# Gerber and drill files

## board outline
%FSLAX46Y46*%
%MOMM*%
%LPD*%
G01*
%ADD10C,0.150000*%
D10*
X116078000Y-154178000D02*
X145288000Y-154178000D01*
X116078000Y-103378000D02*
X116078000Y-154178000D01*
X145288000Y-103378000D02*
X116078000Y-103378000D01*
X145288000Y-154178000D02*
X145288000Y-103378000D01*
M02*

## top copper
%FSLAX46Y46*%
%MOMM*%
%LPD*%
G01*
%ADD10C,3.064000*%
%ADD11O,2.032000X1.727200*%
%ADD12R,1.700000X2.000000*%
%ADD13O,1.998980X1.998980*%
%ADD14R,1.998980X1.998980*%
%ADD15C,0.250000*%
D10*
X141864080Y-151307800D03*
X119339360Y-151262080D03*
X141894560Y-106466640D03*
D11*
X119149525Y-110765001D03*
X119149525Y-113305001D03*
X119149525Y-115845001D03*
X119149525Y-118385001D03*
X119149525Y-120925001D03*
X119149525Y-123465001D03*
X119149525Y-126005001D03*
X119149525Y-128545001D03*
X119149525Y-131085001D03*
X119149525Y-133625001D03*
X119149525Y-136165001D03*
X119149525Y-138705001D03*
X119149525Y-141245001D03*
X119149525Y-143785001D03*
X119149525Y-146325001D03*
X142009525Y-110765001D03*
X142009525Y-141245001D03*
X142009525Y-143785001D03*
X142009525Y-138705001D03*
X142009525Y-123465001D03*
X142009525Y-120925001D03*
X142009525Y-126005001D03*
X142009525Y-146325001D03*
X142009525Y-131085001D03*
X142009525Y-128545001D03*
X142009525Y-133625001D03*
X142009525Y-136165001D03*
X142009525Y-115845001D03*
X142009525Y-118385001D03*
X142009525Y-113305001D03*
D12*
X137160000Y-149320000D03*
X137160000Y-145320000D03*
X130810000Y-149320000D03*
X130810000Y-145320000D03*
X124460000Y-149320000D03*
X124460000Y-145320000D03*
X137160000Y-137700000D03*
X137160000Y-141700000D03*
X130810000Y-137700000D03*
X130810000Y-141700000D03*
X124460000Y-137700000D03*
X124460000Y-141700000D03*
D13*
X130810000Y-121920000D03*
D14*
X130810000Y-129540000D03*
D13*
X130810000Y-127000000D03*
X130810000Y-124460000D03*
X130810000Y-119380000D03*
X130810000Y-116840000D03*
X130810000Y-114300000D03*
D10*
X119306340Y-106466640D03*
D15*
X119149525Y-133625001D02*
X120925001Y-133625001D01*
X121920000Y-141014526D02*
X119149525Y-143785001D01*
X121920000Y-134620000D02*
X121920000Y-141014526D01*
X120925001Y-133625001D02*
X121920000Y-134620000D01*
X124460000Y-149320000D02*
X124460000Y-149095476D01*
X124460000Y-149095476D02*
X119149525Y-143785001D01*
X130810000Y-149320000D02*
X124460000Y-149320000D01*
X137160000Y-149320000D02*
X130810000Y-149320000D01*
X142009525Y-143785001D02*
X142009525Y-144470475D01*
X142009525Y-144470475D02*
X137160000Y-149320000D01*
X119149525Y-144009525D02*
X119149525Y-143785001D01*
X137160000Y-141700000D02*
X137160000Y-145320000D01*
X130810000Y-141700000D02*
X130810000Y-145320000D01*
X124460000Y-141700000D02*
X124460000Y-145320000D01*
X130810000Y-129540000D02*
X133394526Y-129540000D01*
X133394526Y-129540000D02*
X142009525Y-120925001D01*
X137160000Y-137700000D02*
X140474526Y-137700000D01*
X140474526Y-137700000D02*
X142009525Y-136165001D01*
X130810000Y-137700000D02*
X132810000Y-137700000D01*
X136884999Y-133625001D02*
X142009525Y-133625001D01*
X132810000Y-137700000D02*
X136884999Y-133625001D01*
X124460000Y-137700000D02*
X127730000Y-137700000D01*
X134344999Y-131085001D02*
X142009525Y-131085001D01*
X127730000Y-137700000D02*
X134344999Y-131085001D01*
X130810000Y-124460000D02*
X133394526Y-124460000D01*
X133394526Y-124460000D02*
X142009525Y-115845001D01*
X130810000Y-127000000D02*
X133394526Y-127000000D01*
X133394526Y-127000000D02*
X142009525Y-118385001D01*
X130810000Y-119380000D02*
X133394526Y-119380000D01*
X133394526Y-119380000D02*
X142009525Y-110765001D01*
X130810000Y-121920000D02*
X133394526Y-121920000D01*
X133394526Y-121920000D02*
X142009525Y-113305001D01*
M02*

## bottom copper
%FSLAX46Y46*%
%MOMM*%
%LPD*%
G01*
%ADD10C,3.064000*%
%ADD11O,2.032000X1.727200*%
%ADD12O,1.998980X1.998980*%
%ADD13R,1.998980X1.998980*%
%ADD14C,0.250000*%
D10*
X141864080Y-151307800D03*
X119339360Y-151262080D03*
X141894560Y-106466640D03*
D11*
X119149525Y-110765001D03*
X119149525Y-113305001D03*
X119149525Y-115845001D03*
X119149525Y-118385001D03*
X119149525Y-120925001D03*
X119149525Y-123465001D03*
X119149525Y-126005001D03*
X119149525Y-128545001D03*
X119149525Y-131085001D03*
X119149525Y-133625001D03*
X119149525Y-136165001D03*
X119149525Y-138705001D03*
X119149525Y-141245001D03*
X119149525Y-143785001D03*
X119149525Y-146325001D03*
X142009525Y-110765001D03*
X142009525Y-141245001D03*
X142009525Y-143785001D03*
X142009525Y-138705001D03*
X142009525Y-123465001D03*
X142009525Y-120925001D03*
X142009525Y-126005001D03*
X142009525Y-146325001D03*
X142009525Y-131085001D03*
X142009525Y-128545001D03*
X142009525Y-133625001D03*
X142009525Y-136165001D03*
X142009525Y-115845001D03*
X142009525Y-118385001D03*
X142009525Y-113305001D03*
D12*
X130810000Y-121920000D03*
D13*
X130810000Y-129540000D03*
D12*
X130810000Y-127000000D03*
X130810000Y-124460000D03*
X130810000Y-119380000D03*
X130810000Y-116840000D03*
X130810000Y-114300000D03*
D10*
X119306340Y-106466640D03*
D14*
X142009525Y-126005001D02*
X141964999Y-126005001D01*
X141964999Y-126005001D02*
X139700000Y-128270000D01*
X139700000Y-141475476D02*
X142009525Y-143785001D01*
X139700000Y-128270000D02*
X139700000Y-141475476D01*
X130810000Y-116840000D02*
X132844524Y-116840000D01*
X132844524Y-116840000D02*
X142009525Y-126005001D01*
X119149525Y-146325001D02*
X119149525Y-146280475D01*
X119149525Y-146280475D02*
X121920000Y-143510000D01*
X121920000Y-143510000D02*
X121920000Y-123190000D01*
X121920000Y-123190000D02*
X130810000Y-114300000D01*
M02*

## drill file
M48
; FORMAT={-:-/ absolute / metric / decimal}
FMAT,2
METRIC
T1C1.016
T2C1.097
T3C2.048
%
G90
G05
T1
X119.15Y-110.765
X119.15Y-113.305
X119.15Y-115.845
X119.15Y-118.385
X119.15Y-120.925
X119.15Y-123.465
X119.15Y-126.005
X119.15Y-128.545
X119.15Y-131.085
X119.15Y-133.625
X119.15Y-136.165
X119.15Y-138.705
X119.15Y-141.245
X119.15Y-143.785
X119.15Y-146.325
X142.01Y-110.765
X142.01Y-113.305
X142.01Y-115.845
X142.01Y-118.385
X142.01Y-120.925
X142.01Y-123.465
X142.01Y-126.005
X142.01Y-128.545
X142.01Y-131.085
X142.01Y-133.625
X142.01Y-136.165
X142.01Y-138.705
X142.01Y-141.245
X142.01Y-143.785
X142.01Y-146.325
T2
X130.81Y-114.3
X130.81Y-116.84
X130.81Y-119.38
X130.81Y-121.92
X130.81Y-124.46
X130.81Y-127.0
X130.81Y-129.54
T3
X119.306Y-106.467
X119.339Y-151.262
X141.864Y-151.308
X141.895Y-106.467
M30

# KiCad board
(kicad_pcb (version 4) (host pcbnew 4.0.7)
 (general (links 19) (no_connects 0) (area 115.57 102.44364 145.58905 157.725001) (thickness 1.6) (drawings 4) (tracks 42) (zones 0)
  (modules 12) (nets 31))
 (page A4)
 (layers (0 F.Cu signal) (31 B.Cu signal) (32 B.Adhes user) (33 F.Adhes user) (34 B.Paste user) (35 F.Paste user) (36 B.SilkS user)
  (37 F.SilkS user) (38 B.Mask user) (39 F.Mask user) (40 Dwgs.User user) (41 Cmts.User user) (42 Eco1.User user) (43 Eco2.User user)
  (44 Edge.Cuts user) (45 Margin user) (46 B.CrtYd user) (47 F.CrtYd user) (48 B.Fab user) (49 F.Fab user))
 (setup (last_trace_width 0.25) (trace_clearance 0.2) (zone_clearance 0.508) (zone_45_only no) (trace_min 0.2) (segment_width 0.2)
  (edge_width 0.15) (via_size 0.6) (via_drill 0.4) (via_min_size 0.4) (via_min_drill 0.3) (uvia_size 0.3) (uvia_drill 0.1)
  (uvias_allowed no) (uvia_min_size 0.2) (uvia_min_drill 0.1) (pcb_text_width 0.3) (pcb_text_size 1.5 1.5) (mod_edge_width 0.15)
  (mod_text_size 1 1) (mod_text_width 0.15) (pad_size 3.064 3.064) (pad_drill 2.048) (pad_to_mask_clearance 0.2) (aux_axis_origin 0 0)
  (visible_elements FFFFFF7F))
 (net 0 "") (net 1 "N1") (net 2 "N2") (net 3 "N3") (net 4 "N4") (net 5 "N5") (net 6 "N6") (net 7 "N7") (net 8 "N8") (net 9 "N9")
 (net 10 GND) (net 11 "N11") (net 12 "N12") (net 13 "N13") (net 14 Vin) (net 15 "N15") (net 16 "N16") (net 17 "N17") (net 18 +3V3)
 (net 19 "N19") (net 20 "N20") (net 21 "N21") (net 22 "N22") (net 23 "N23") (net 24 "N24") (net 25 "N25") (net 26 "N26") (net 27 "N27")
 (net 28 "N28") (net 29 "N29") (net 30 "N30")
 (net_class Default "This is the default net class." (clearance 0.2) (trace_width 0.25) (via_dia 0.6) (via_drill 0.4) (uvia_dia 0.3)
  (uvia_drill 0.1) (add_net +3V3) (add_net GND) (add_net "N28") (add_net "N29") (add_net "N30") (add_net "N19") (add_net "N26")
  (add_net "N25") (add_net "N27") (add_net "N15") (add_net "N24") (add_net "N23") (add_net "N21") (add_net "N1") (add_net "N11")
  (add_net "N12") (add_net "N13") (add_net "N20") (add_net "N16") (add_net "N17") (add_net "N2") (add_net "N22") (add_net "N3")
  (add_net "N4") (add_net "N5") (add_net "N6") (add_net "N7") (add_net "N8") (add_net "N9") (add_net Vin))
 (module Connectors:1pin (layer F.Cu) (at 141.86408 151.3078)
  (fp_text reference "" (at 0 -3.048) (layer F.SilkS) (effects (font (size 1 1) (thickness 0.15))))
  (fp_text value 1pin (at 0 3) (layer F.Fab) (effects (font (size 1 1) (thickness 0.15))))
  (pad 1 thru_hole circle (at 0 0) (size 3.064 3.064) (drill 2.048) (layers *.Cu *.Mask)))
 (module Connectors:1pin (layer F.Cu) (at 119.33936 151.26208)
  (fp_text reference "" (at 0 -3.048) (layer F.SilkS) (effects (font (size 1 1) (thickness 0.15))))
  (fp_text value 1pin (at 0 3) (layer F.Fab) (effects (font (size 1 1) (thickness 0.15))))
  (pad 1 thru_hole circle (at 0 0) (size 3.064 3.064) (drill 2.048) (layers *.Cu *.Mask)))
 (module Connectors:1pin (layer F.Cu) (at 141.89456 106.46664)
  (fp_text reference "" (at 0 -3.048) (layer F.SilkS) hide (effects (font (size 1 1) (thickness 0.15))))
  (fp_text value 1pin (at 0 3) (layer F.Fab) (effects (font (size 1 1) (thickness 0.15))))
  (pad 1 thru_hole circle (at 0 0) (size 3.064 3.064) (drill 2.048) (layers *.Cu *.Mask)))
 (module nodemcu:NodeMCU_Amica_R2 (layer F.Cu) (at 119.149525 110.765001)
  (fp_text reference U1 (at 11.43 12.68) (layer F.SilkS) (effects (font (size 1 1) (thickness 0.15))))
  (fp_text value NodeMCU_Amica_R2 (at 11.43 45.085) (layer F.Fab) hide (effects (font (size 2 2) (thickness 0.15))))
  (pad 1 thru_hole oval (at 0 0) (size 2.032 1.7272) (drill 1.016) (layers *.Cu *.Mask F.SilkS) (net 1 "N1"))
  (pad 2 thru_hole oval (at 0 2.54) (size 2.032 1.7272) (drill 1.016) (layers *.Cu *.Mask F.SilkS) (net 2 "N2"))
  (pad 3 thru_hole oval (at 0 5.08) (size 2.032 1.7272) (drill 1.016) (layers *.Cu *.Mask F.SilkS) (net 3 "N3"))
  (pad 4 thru_hole oval (at 0 7.62) (size 2.032 1.7272) (drill 1.016) (layers *.Cu *.Mask F.SilkS) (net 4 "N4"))
  (pad 5 thru_hole oval (at 0 10.16) (size 2.032 1.7272) (drill 1.016) (layers *.Cu *.Mask F.SilkS) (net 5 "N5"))
  (pad 6 thru_hole oval (at 0 12.7) (size 2.032 1.7272) (drill 1.016) (layers *.Cu *.Mask F.SilkS) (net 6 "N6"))
  (pad 7 thru_hole oval (at 0 15.24) (size 2.032 1.7272) (drill 1.016) (layers *.Cu *.Mask F.SilkS) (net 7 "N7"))
  (pad 8 thru_hole oval (at 0 17.78) (size 2.032 1.7272) (drill 1.016) (layers *.Cu *.Mask F.SilkS) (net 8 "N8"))
  (pad 9 thru_hole oval (at 0 20.32) (size 2.032 1.7272) (drill 1.016) (layers *.Cu *.Mask F.SilkS) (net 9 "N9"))
  (pad 10 thru_hole oval (at 0 22.86) (size 2.032 1.7272) (drill 1.016) (layers *.Cu *.Mask F.SilkS) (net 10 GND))
  (pad 11 thru_hole oval (at 0 25.4) (size 2.032 1.7272) (drill 1.016) (layers *.Cu *.Mask F.SilkS) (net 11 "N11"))
  (pad 12 thru_hole oval (at 0 27.94) (size 2.032 1.7272) (drill 1.016) (layers *.Cu *.Mask F.SilkS) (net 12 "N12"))
  (pad 13 thru_hole oval (at 0 30.48) (size 2.032 1.7272) (drill 1.016) (layers *.Cu *.Mask F.SilkS) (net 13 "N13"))
  (pad 14 thru_hole oval (at 0 33.02) (size 2.032 1.7272) (drill 1.016) (layers *.Cu *.Mask F.SilkS) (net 10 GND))
  (pad 15 thru_hole oval (at 0 35.56) (size 2.032 1.7272) (drill 1.016) (layers *.Cu *.Mask F.SilkS) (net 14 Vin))
  (pad 30 thru_hole oval (at 22.86 0) (size 2.032 1.7272) (drill 1.016) (layers *.Cu *.Mask F.SilkS) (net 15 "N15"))
  (pad 18 thru_hole oval (at 22.86 30.48) (size 2.032 1.7272) (drill 1.016) (layers *.Cu *.Mask F.SilkS) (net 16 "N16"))
  (pad 17 thru_hole oval (at 22.86 33.02) (size 2.032 1.7272) (drill 1.016) (layers *.Cu *.Mask F.SilkS) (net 10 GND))
  (pad 19 thru_hole oval (at 22.86 27.94) (size 2.032 1.7272) (drill 1.016) (layers *.Cu *.Mask F.SilkS) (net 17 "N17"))
  (pad 25 thru_hole oval (at 22.86 12.7) (size 2.032 1.7272) (drill 1.016) (layers *.Cu *.Mask F.SilkS) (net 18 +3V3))
  (pad 26 thru_hole oval (at 22.86 10.16) (size 2.032 1.7272) (drill 1.016) (layers *.Cu *.Mask F.SilkS) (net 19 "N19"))
  (pad 24 thru_hole oval (at 22.86 15.24) (size 2.032 1.7272) (drill 1.016) (layers *.Cu *.Mask F.SilkS) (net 10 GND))
  (pad 16 thru_hole oval (at 22.86 35.56) (size 2.032 1.7272) (drill 1.016) (layers *.Cu *.Mask F.SilkS) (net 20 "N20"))
  (pad 22 thru_hole oval (at 22.86 20.32) (size 2.032 1.7272) (drill 1.016) (layers *.Cu *.Mask F.SilkS) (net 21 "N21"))
  (pad 23 thru_hole oval (at 22.86 17.78) (size 2.032 1.7272) (drill 1.016) (layers *.Cu *.Mask F.SilkS) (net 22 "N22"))
  (pad 21 thru_hole oval (at 22.86 22.86) (size 2.032 1.7272) (drill 1.016) (layers *.Cu *.Mask F.SilkS) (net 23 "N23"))
  (pad 20 thru_hole oval (at 22.86 25.4) (size 2.032 1.7272) (drill 1.016) (layers *.Cu *.Mask F.SilkS) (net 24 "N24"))
  (pad 28 thru_hole oval (at 22.86 5.08) (size 2.032 1.7272) (drill 1.016) (layers *.Cu *.Mask F.SilkS) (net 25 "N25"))
  (pad 27 thru_hole oval (at 22.86 7.62) (size 2.032 1.7272) (drill 1.016) (layers *.Cu *.Mask F.SilkS) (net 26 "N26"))
  (pad 29 thru_hole oval (at 22.86 2.54) (size 2.032 1.7272) (drill 1.016) (layers *.Cu *.Mask F.SilkS) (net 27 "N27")))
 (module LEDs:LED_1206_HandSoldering (layer F.Cu) (at 137.16 147.32 90)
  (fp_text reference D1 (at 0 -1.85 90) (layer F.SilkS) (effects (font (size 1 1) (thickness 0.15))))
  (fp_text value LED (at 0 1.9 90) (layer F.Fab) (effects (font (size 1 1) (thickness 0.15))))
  (pad 1 smd rect (at -2 0 90) (size 2 1.7) (layers F.Cu F.Paste F.Mask) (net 10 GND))
  (pad 2 smd rect (at 2 0 90) (size 2 1.7) (layers F.Cu F.Paste F.Mask) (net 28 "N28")))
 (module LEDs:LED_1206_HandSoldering (layer F.Cu) (at 130.81 147.32 90)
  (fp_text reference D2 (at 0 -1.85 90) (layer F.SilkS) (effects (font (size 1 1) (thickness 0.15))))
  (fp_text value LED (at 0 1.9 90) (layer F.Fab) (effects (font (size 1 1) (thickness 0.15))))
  (pad 1 smd rect (at -2 0 90) (size 2 1.7) (layers F.Cu F.Paste F.Mask) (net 10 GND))
  (pad 2 smd rect (at 2 0 90) (size 2 1.7) (layers F.Cu F.Paste F.Mask) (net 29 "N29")))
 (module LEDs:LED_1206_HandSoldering (layer F.Cu) (at 124.46 147.32 90)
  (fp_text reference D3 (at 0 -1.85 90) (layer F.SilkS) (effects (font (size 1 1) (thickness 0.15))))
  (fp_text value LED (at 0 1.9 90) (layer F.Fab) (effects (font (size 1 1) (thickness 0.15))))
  (pad 1 smd rect (at -2 0 90) (size 2 1.7) (layers F.Cu F.Paste F.Mask) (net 10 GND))
  (pad 2 smd rect (at 2 0 90) (size 2 1.7) (layers F.Cu F.Paste F.Mask) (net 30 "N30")))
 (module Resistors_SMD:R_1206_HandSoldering (layer F.Cu) (at 137.16 139.7 270)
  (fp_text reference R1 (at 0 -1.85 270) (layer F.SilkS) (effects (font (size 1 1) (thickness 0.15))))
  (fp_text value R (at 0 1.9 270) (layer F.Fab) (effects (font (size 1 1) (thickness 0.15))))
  (pad 1 smd rect (at -2 0 270) (size 2 1.7) (layers F.Cu F.Paste F.Mask) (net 24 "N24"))
  (pad 2 smd rect (at 2 0 270) (size 2 1.7) (layers F.Cu F.Paste F.Mask) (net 28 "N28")))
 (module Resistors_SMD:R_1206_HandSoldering (layer F.Cu) (at 130.81 139.7 270)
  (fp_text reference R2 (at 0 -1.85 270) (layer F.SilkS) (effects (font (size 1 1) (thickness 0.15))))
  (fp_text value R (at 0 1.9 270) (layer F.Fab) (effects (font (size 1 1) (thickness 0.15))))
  (pad 1 smd rect (at -2 0 270) (size 2 1.7) (layers F.Cu F.Paste F.Mask) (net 23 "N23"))
  (pad 2 smd rect (at 2 0 270) (size 2 1.7) (layers F.Cu F.Paste F.Mask) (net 29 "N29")))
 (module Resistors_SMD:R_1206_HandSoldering (layer F.Cu) (at 124.46 139.7 270)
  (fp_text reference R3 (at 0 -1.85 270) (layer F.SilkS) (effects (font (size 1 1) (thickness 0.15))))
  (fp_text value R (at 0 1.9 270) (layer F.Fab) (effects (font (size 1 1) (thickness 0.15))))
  (pad 1 smd rect (at -2 0 270) (size 2 1.7) (layers F.Cu F.Paste F.Mask) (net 21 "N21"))
  (pad 2 smd rect (at 2 0 270) (size 2 1.7) (layers F.Cu F.Paste F.Mask) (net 30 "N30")))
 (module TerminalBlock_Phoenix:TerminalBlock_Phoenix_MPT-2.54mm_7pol (layer F.Cu) (at 130.81 129.54 90)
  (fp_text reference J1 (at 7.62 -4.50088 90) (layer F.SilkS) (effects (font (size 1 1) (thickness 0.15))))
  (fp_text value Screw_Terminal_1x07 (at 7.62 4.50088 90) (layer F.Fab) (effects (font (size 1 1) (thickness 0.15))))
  (pad 4 thru_hole oval (at 7.62 0 270) (size 1.99898 1.99898) (drill 1.09728) (layers *.Cu *.Mask) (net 27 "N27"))
  (pad 1 thru_hole rect (at 0 0 270) (size 1.99898 1.99898) (drill 1.09728) (layers *.Cu *.Mask) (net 19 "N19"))
  (pad 2 thru_hole oval (at 2.54 0 270) (size 1.99898 1.99898) (drill 1.09728) (layers *.Cu *.Mask) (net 26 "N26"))
  (pad 3 thru_hole oval (at 5.08 0 270) (size 1.99898 1.99898) (drill 1.09728) (layers *.Cu *.Mask) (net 25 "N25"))
  (pad 5 thru_hole oval (at 10.16 0 270) (size 1.99898 1.99898) (drill 1.09728) (layers *.Cu *.Mask) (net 15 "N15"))
  (pad 6 thru_hole oval (at 12.7 0 270) (size 1.99898 1.99898) (drill 1.09728) (layers *.Cu *.Mask) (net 10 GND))
  (pad 7 thru_hole oval (at 15.24 0 270) (size 1.99898 1.99898) (drill 1.09728) (layers *.Cu *.Mask) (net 14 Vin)))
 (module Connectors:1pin (layer F.Cu) (at 119.30634 106.46664)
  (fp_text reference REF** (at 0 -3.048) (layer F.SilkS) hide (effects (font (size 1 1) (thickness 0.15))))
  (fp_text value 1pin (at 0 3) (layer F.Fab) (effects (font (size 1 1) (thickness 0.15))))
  (pad 1 thru_hole circle (at 0 0) (size 3.064 3.064) (drill 2.048) (layers *.Cu *.Mask)))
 (gr_line (start 116.078 154.178) (end 145.288 154.178) (angle 90) (layer Edge.Cuts) (width 0.15))
 (gr_line (start 116.078 103.378) (end 116.078 154.178) (angle 90) (layer Edge.Cuts) (width 0.15))
 (gr_line (start 145.288 103.378) (end 116.078 103.378) (angle 90) (layer Edge.Cuts) (width 0.15))
 (gr_line (start 145.288 154.178) (end 145.288 103.378) (angle 90) (layer Edge.Cuts) (width 0.15))
 (segment (start 142.009525 126.005001) (end 141.964999 126.005001) (width 0.25) (layer B.Cu) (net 10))
 (segment (start 141.964999 126.005001) (end 139.7 128.27) (width 0.25) (layer B.Cu) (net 10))
 (segment (start 139.7 141.475476) (end 142.009525 143.785001) (width 0.25) (layer B.Cu) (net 10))
 (segment (start 139.7 128.27) (end 139.7 141.475476) (width 0.25) (layer B.Cu) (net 10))
 (segment (start 119.149525 133.625001) (end 120.925001 133.625001) (width 0.25) (layer F.Cu) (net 10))
 (segment (start 121.92 141.014526) (end 119.149525 143.785001) (width 0.25) (layer F.Cu) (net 10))
 (segment (start 121.92 134.62) (end 121.92 141.014526) (width 0.25) (layer F.Cu) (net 10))
 (segment (start 120.925001 133.625001) (end 121.92 134.62) (width 0.25) (layer F.Cu) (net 10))
 (segment (start 130.81 116.84) (end 132.844524 116.84) (width 0.25) (layer B.Cu) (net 10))
 (segment (start 132.844524 116.84) (end 142.009525 126.005001) (width 0.25) (layer B.Cu) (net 10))
 (segment (start 124.46 149.32) (end 124.46 149.095476) (width 0.25) (layer F.Cu) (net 10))
 (segment (start 124.46 149.095476) (end 119.149525 143.785001) (width 0.25) (layer F.Cu) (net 10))
 (segment (start 130.81 149.32) (end 124.46 149.32) (width 0.25) (layer F.Cu) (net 10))
 (segment (start 137.16 149.32) (end 130.81 149.32) (width 0.25) (layer F.Cu) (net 10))
 (segment (start 142.009525 143.785001) (end 142.009525 144.470475) (width 0.25) (layer F.Cu) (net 10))
 (segment (start 142.009525 144.470475) (end 137.16 149.32) (width 0.25) (layer F.Cu) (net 10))
 (segment (start 119.149525 144.009525) (end 119.149525 143.785001) (width 0.25) (layer F.Cu) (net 10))
 (segment (start 137.16 141.7) (end 137.16 145.32) (width 0.25) (layer F.Cu) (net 28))
 (segment (start 130.81 141.7) (end 130.81 145.32) (width 0.25) (layer F.Cu) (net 29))
 (segment (start 124.46 141.7) (end 124.46 145.32) (width 0.25) (layer F.Cu) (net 30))
 (segment (start 119.149525 146.325001) (end 119.149525 146.280475) (width 0.25) (layer B.Cu) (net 14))
 (segment (start 119.149525 146.280475) (end 121.92 143.51) (width 0.25) (layer B.Cu) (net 14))
 (segment (start 121.92 143.51) (end 121.92 123.19) (width 0.25) (layer B.Cu) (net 14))
 (segment (start 121.92 123.19) (end 130.81 114.3) (width 0.25) (layer B.Cu) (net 14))
 (segment (start 130.81 129.54) (end 133.394526 129.54) (width 0.25) (layer F.Cu) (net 19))
 (segment (start 133.394526 129.54) (end 142.009525 120.925001) (width 0.25) (layer F.Cu) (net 19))
 (segment (start 137.16 137.7) (end 140.474526 137.7) (width 0.25) (layer F.Cu) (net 24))
 (segment (start 140.474526 137.7) (end 142.009525 136.165001) (width 0.25) (layer F.Cu) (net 24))
 (segment (start 130.81 137.7) (end 132.81 137.7) (width 0.25) (layer F.Cu) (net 23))
 (segment (start 136.884999 133.625001) (end 142.009525 133.625001) (width 0.25) (layer F.Cu) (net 23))
 (segment (start 132.81 137.7) (end 136.884999 133.625001) (width 0.25) (layer F.Cu) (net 23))
 (segment (start 124.46 137.7) (end 127.73 137.7) (width 0.25) (layer F.Cu) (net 21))
 (segment (start 134.344999 131.085001) (end 142.009525 131.085001) (width 0.25) (layer F.Cu) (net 21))
 (segment (start 127.73 137.7) (end 134.344999 131.085001) (width 0.25) (layer F.Cu) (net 21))
 (segment (start 130.81 124.46) (end 133.394526 124.46) (width 0.25) (layer F.Cu) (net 25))
 (segment (start 133.394526 124.46) (end 142.009525 115.845001) (width 0.25) (layer F.Cu) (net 25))
 (segment (start 130.81 127) (end 133.394526 127) (width 0.25) (layer F.Cu) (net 26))
 (segment (start 133.394526 127) (end 142.009525 118.385001) (width 0.25) (layer F.Cu) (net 26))
 (segment (start 130.81 119.38) (end 133.394526 119.38) (width 0.25) (layer F.Cu) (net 15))
 (segment (start 133.394526 119.38) (end 142.009525 110.765001) (width 0.25) (layer F.Cu) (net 15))
 (segment (start 130.81 121.92) (end 133.394526 121.92) (width 0.25) (layer F.Cu) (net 27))
 (segment (start 133.394526 121.92) (end 142.009525 113.305001) (width 0.25) (layer F.Cu) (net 27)))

